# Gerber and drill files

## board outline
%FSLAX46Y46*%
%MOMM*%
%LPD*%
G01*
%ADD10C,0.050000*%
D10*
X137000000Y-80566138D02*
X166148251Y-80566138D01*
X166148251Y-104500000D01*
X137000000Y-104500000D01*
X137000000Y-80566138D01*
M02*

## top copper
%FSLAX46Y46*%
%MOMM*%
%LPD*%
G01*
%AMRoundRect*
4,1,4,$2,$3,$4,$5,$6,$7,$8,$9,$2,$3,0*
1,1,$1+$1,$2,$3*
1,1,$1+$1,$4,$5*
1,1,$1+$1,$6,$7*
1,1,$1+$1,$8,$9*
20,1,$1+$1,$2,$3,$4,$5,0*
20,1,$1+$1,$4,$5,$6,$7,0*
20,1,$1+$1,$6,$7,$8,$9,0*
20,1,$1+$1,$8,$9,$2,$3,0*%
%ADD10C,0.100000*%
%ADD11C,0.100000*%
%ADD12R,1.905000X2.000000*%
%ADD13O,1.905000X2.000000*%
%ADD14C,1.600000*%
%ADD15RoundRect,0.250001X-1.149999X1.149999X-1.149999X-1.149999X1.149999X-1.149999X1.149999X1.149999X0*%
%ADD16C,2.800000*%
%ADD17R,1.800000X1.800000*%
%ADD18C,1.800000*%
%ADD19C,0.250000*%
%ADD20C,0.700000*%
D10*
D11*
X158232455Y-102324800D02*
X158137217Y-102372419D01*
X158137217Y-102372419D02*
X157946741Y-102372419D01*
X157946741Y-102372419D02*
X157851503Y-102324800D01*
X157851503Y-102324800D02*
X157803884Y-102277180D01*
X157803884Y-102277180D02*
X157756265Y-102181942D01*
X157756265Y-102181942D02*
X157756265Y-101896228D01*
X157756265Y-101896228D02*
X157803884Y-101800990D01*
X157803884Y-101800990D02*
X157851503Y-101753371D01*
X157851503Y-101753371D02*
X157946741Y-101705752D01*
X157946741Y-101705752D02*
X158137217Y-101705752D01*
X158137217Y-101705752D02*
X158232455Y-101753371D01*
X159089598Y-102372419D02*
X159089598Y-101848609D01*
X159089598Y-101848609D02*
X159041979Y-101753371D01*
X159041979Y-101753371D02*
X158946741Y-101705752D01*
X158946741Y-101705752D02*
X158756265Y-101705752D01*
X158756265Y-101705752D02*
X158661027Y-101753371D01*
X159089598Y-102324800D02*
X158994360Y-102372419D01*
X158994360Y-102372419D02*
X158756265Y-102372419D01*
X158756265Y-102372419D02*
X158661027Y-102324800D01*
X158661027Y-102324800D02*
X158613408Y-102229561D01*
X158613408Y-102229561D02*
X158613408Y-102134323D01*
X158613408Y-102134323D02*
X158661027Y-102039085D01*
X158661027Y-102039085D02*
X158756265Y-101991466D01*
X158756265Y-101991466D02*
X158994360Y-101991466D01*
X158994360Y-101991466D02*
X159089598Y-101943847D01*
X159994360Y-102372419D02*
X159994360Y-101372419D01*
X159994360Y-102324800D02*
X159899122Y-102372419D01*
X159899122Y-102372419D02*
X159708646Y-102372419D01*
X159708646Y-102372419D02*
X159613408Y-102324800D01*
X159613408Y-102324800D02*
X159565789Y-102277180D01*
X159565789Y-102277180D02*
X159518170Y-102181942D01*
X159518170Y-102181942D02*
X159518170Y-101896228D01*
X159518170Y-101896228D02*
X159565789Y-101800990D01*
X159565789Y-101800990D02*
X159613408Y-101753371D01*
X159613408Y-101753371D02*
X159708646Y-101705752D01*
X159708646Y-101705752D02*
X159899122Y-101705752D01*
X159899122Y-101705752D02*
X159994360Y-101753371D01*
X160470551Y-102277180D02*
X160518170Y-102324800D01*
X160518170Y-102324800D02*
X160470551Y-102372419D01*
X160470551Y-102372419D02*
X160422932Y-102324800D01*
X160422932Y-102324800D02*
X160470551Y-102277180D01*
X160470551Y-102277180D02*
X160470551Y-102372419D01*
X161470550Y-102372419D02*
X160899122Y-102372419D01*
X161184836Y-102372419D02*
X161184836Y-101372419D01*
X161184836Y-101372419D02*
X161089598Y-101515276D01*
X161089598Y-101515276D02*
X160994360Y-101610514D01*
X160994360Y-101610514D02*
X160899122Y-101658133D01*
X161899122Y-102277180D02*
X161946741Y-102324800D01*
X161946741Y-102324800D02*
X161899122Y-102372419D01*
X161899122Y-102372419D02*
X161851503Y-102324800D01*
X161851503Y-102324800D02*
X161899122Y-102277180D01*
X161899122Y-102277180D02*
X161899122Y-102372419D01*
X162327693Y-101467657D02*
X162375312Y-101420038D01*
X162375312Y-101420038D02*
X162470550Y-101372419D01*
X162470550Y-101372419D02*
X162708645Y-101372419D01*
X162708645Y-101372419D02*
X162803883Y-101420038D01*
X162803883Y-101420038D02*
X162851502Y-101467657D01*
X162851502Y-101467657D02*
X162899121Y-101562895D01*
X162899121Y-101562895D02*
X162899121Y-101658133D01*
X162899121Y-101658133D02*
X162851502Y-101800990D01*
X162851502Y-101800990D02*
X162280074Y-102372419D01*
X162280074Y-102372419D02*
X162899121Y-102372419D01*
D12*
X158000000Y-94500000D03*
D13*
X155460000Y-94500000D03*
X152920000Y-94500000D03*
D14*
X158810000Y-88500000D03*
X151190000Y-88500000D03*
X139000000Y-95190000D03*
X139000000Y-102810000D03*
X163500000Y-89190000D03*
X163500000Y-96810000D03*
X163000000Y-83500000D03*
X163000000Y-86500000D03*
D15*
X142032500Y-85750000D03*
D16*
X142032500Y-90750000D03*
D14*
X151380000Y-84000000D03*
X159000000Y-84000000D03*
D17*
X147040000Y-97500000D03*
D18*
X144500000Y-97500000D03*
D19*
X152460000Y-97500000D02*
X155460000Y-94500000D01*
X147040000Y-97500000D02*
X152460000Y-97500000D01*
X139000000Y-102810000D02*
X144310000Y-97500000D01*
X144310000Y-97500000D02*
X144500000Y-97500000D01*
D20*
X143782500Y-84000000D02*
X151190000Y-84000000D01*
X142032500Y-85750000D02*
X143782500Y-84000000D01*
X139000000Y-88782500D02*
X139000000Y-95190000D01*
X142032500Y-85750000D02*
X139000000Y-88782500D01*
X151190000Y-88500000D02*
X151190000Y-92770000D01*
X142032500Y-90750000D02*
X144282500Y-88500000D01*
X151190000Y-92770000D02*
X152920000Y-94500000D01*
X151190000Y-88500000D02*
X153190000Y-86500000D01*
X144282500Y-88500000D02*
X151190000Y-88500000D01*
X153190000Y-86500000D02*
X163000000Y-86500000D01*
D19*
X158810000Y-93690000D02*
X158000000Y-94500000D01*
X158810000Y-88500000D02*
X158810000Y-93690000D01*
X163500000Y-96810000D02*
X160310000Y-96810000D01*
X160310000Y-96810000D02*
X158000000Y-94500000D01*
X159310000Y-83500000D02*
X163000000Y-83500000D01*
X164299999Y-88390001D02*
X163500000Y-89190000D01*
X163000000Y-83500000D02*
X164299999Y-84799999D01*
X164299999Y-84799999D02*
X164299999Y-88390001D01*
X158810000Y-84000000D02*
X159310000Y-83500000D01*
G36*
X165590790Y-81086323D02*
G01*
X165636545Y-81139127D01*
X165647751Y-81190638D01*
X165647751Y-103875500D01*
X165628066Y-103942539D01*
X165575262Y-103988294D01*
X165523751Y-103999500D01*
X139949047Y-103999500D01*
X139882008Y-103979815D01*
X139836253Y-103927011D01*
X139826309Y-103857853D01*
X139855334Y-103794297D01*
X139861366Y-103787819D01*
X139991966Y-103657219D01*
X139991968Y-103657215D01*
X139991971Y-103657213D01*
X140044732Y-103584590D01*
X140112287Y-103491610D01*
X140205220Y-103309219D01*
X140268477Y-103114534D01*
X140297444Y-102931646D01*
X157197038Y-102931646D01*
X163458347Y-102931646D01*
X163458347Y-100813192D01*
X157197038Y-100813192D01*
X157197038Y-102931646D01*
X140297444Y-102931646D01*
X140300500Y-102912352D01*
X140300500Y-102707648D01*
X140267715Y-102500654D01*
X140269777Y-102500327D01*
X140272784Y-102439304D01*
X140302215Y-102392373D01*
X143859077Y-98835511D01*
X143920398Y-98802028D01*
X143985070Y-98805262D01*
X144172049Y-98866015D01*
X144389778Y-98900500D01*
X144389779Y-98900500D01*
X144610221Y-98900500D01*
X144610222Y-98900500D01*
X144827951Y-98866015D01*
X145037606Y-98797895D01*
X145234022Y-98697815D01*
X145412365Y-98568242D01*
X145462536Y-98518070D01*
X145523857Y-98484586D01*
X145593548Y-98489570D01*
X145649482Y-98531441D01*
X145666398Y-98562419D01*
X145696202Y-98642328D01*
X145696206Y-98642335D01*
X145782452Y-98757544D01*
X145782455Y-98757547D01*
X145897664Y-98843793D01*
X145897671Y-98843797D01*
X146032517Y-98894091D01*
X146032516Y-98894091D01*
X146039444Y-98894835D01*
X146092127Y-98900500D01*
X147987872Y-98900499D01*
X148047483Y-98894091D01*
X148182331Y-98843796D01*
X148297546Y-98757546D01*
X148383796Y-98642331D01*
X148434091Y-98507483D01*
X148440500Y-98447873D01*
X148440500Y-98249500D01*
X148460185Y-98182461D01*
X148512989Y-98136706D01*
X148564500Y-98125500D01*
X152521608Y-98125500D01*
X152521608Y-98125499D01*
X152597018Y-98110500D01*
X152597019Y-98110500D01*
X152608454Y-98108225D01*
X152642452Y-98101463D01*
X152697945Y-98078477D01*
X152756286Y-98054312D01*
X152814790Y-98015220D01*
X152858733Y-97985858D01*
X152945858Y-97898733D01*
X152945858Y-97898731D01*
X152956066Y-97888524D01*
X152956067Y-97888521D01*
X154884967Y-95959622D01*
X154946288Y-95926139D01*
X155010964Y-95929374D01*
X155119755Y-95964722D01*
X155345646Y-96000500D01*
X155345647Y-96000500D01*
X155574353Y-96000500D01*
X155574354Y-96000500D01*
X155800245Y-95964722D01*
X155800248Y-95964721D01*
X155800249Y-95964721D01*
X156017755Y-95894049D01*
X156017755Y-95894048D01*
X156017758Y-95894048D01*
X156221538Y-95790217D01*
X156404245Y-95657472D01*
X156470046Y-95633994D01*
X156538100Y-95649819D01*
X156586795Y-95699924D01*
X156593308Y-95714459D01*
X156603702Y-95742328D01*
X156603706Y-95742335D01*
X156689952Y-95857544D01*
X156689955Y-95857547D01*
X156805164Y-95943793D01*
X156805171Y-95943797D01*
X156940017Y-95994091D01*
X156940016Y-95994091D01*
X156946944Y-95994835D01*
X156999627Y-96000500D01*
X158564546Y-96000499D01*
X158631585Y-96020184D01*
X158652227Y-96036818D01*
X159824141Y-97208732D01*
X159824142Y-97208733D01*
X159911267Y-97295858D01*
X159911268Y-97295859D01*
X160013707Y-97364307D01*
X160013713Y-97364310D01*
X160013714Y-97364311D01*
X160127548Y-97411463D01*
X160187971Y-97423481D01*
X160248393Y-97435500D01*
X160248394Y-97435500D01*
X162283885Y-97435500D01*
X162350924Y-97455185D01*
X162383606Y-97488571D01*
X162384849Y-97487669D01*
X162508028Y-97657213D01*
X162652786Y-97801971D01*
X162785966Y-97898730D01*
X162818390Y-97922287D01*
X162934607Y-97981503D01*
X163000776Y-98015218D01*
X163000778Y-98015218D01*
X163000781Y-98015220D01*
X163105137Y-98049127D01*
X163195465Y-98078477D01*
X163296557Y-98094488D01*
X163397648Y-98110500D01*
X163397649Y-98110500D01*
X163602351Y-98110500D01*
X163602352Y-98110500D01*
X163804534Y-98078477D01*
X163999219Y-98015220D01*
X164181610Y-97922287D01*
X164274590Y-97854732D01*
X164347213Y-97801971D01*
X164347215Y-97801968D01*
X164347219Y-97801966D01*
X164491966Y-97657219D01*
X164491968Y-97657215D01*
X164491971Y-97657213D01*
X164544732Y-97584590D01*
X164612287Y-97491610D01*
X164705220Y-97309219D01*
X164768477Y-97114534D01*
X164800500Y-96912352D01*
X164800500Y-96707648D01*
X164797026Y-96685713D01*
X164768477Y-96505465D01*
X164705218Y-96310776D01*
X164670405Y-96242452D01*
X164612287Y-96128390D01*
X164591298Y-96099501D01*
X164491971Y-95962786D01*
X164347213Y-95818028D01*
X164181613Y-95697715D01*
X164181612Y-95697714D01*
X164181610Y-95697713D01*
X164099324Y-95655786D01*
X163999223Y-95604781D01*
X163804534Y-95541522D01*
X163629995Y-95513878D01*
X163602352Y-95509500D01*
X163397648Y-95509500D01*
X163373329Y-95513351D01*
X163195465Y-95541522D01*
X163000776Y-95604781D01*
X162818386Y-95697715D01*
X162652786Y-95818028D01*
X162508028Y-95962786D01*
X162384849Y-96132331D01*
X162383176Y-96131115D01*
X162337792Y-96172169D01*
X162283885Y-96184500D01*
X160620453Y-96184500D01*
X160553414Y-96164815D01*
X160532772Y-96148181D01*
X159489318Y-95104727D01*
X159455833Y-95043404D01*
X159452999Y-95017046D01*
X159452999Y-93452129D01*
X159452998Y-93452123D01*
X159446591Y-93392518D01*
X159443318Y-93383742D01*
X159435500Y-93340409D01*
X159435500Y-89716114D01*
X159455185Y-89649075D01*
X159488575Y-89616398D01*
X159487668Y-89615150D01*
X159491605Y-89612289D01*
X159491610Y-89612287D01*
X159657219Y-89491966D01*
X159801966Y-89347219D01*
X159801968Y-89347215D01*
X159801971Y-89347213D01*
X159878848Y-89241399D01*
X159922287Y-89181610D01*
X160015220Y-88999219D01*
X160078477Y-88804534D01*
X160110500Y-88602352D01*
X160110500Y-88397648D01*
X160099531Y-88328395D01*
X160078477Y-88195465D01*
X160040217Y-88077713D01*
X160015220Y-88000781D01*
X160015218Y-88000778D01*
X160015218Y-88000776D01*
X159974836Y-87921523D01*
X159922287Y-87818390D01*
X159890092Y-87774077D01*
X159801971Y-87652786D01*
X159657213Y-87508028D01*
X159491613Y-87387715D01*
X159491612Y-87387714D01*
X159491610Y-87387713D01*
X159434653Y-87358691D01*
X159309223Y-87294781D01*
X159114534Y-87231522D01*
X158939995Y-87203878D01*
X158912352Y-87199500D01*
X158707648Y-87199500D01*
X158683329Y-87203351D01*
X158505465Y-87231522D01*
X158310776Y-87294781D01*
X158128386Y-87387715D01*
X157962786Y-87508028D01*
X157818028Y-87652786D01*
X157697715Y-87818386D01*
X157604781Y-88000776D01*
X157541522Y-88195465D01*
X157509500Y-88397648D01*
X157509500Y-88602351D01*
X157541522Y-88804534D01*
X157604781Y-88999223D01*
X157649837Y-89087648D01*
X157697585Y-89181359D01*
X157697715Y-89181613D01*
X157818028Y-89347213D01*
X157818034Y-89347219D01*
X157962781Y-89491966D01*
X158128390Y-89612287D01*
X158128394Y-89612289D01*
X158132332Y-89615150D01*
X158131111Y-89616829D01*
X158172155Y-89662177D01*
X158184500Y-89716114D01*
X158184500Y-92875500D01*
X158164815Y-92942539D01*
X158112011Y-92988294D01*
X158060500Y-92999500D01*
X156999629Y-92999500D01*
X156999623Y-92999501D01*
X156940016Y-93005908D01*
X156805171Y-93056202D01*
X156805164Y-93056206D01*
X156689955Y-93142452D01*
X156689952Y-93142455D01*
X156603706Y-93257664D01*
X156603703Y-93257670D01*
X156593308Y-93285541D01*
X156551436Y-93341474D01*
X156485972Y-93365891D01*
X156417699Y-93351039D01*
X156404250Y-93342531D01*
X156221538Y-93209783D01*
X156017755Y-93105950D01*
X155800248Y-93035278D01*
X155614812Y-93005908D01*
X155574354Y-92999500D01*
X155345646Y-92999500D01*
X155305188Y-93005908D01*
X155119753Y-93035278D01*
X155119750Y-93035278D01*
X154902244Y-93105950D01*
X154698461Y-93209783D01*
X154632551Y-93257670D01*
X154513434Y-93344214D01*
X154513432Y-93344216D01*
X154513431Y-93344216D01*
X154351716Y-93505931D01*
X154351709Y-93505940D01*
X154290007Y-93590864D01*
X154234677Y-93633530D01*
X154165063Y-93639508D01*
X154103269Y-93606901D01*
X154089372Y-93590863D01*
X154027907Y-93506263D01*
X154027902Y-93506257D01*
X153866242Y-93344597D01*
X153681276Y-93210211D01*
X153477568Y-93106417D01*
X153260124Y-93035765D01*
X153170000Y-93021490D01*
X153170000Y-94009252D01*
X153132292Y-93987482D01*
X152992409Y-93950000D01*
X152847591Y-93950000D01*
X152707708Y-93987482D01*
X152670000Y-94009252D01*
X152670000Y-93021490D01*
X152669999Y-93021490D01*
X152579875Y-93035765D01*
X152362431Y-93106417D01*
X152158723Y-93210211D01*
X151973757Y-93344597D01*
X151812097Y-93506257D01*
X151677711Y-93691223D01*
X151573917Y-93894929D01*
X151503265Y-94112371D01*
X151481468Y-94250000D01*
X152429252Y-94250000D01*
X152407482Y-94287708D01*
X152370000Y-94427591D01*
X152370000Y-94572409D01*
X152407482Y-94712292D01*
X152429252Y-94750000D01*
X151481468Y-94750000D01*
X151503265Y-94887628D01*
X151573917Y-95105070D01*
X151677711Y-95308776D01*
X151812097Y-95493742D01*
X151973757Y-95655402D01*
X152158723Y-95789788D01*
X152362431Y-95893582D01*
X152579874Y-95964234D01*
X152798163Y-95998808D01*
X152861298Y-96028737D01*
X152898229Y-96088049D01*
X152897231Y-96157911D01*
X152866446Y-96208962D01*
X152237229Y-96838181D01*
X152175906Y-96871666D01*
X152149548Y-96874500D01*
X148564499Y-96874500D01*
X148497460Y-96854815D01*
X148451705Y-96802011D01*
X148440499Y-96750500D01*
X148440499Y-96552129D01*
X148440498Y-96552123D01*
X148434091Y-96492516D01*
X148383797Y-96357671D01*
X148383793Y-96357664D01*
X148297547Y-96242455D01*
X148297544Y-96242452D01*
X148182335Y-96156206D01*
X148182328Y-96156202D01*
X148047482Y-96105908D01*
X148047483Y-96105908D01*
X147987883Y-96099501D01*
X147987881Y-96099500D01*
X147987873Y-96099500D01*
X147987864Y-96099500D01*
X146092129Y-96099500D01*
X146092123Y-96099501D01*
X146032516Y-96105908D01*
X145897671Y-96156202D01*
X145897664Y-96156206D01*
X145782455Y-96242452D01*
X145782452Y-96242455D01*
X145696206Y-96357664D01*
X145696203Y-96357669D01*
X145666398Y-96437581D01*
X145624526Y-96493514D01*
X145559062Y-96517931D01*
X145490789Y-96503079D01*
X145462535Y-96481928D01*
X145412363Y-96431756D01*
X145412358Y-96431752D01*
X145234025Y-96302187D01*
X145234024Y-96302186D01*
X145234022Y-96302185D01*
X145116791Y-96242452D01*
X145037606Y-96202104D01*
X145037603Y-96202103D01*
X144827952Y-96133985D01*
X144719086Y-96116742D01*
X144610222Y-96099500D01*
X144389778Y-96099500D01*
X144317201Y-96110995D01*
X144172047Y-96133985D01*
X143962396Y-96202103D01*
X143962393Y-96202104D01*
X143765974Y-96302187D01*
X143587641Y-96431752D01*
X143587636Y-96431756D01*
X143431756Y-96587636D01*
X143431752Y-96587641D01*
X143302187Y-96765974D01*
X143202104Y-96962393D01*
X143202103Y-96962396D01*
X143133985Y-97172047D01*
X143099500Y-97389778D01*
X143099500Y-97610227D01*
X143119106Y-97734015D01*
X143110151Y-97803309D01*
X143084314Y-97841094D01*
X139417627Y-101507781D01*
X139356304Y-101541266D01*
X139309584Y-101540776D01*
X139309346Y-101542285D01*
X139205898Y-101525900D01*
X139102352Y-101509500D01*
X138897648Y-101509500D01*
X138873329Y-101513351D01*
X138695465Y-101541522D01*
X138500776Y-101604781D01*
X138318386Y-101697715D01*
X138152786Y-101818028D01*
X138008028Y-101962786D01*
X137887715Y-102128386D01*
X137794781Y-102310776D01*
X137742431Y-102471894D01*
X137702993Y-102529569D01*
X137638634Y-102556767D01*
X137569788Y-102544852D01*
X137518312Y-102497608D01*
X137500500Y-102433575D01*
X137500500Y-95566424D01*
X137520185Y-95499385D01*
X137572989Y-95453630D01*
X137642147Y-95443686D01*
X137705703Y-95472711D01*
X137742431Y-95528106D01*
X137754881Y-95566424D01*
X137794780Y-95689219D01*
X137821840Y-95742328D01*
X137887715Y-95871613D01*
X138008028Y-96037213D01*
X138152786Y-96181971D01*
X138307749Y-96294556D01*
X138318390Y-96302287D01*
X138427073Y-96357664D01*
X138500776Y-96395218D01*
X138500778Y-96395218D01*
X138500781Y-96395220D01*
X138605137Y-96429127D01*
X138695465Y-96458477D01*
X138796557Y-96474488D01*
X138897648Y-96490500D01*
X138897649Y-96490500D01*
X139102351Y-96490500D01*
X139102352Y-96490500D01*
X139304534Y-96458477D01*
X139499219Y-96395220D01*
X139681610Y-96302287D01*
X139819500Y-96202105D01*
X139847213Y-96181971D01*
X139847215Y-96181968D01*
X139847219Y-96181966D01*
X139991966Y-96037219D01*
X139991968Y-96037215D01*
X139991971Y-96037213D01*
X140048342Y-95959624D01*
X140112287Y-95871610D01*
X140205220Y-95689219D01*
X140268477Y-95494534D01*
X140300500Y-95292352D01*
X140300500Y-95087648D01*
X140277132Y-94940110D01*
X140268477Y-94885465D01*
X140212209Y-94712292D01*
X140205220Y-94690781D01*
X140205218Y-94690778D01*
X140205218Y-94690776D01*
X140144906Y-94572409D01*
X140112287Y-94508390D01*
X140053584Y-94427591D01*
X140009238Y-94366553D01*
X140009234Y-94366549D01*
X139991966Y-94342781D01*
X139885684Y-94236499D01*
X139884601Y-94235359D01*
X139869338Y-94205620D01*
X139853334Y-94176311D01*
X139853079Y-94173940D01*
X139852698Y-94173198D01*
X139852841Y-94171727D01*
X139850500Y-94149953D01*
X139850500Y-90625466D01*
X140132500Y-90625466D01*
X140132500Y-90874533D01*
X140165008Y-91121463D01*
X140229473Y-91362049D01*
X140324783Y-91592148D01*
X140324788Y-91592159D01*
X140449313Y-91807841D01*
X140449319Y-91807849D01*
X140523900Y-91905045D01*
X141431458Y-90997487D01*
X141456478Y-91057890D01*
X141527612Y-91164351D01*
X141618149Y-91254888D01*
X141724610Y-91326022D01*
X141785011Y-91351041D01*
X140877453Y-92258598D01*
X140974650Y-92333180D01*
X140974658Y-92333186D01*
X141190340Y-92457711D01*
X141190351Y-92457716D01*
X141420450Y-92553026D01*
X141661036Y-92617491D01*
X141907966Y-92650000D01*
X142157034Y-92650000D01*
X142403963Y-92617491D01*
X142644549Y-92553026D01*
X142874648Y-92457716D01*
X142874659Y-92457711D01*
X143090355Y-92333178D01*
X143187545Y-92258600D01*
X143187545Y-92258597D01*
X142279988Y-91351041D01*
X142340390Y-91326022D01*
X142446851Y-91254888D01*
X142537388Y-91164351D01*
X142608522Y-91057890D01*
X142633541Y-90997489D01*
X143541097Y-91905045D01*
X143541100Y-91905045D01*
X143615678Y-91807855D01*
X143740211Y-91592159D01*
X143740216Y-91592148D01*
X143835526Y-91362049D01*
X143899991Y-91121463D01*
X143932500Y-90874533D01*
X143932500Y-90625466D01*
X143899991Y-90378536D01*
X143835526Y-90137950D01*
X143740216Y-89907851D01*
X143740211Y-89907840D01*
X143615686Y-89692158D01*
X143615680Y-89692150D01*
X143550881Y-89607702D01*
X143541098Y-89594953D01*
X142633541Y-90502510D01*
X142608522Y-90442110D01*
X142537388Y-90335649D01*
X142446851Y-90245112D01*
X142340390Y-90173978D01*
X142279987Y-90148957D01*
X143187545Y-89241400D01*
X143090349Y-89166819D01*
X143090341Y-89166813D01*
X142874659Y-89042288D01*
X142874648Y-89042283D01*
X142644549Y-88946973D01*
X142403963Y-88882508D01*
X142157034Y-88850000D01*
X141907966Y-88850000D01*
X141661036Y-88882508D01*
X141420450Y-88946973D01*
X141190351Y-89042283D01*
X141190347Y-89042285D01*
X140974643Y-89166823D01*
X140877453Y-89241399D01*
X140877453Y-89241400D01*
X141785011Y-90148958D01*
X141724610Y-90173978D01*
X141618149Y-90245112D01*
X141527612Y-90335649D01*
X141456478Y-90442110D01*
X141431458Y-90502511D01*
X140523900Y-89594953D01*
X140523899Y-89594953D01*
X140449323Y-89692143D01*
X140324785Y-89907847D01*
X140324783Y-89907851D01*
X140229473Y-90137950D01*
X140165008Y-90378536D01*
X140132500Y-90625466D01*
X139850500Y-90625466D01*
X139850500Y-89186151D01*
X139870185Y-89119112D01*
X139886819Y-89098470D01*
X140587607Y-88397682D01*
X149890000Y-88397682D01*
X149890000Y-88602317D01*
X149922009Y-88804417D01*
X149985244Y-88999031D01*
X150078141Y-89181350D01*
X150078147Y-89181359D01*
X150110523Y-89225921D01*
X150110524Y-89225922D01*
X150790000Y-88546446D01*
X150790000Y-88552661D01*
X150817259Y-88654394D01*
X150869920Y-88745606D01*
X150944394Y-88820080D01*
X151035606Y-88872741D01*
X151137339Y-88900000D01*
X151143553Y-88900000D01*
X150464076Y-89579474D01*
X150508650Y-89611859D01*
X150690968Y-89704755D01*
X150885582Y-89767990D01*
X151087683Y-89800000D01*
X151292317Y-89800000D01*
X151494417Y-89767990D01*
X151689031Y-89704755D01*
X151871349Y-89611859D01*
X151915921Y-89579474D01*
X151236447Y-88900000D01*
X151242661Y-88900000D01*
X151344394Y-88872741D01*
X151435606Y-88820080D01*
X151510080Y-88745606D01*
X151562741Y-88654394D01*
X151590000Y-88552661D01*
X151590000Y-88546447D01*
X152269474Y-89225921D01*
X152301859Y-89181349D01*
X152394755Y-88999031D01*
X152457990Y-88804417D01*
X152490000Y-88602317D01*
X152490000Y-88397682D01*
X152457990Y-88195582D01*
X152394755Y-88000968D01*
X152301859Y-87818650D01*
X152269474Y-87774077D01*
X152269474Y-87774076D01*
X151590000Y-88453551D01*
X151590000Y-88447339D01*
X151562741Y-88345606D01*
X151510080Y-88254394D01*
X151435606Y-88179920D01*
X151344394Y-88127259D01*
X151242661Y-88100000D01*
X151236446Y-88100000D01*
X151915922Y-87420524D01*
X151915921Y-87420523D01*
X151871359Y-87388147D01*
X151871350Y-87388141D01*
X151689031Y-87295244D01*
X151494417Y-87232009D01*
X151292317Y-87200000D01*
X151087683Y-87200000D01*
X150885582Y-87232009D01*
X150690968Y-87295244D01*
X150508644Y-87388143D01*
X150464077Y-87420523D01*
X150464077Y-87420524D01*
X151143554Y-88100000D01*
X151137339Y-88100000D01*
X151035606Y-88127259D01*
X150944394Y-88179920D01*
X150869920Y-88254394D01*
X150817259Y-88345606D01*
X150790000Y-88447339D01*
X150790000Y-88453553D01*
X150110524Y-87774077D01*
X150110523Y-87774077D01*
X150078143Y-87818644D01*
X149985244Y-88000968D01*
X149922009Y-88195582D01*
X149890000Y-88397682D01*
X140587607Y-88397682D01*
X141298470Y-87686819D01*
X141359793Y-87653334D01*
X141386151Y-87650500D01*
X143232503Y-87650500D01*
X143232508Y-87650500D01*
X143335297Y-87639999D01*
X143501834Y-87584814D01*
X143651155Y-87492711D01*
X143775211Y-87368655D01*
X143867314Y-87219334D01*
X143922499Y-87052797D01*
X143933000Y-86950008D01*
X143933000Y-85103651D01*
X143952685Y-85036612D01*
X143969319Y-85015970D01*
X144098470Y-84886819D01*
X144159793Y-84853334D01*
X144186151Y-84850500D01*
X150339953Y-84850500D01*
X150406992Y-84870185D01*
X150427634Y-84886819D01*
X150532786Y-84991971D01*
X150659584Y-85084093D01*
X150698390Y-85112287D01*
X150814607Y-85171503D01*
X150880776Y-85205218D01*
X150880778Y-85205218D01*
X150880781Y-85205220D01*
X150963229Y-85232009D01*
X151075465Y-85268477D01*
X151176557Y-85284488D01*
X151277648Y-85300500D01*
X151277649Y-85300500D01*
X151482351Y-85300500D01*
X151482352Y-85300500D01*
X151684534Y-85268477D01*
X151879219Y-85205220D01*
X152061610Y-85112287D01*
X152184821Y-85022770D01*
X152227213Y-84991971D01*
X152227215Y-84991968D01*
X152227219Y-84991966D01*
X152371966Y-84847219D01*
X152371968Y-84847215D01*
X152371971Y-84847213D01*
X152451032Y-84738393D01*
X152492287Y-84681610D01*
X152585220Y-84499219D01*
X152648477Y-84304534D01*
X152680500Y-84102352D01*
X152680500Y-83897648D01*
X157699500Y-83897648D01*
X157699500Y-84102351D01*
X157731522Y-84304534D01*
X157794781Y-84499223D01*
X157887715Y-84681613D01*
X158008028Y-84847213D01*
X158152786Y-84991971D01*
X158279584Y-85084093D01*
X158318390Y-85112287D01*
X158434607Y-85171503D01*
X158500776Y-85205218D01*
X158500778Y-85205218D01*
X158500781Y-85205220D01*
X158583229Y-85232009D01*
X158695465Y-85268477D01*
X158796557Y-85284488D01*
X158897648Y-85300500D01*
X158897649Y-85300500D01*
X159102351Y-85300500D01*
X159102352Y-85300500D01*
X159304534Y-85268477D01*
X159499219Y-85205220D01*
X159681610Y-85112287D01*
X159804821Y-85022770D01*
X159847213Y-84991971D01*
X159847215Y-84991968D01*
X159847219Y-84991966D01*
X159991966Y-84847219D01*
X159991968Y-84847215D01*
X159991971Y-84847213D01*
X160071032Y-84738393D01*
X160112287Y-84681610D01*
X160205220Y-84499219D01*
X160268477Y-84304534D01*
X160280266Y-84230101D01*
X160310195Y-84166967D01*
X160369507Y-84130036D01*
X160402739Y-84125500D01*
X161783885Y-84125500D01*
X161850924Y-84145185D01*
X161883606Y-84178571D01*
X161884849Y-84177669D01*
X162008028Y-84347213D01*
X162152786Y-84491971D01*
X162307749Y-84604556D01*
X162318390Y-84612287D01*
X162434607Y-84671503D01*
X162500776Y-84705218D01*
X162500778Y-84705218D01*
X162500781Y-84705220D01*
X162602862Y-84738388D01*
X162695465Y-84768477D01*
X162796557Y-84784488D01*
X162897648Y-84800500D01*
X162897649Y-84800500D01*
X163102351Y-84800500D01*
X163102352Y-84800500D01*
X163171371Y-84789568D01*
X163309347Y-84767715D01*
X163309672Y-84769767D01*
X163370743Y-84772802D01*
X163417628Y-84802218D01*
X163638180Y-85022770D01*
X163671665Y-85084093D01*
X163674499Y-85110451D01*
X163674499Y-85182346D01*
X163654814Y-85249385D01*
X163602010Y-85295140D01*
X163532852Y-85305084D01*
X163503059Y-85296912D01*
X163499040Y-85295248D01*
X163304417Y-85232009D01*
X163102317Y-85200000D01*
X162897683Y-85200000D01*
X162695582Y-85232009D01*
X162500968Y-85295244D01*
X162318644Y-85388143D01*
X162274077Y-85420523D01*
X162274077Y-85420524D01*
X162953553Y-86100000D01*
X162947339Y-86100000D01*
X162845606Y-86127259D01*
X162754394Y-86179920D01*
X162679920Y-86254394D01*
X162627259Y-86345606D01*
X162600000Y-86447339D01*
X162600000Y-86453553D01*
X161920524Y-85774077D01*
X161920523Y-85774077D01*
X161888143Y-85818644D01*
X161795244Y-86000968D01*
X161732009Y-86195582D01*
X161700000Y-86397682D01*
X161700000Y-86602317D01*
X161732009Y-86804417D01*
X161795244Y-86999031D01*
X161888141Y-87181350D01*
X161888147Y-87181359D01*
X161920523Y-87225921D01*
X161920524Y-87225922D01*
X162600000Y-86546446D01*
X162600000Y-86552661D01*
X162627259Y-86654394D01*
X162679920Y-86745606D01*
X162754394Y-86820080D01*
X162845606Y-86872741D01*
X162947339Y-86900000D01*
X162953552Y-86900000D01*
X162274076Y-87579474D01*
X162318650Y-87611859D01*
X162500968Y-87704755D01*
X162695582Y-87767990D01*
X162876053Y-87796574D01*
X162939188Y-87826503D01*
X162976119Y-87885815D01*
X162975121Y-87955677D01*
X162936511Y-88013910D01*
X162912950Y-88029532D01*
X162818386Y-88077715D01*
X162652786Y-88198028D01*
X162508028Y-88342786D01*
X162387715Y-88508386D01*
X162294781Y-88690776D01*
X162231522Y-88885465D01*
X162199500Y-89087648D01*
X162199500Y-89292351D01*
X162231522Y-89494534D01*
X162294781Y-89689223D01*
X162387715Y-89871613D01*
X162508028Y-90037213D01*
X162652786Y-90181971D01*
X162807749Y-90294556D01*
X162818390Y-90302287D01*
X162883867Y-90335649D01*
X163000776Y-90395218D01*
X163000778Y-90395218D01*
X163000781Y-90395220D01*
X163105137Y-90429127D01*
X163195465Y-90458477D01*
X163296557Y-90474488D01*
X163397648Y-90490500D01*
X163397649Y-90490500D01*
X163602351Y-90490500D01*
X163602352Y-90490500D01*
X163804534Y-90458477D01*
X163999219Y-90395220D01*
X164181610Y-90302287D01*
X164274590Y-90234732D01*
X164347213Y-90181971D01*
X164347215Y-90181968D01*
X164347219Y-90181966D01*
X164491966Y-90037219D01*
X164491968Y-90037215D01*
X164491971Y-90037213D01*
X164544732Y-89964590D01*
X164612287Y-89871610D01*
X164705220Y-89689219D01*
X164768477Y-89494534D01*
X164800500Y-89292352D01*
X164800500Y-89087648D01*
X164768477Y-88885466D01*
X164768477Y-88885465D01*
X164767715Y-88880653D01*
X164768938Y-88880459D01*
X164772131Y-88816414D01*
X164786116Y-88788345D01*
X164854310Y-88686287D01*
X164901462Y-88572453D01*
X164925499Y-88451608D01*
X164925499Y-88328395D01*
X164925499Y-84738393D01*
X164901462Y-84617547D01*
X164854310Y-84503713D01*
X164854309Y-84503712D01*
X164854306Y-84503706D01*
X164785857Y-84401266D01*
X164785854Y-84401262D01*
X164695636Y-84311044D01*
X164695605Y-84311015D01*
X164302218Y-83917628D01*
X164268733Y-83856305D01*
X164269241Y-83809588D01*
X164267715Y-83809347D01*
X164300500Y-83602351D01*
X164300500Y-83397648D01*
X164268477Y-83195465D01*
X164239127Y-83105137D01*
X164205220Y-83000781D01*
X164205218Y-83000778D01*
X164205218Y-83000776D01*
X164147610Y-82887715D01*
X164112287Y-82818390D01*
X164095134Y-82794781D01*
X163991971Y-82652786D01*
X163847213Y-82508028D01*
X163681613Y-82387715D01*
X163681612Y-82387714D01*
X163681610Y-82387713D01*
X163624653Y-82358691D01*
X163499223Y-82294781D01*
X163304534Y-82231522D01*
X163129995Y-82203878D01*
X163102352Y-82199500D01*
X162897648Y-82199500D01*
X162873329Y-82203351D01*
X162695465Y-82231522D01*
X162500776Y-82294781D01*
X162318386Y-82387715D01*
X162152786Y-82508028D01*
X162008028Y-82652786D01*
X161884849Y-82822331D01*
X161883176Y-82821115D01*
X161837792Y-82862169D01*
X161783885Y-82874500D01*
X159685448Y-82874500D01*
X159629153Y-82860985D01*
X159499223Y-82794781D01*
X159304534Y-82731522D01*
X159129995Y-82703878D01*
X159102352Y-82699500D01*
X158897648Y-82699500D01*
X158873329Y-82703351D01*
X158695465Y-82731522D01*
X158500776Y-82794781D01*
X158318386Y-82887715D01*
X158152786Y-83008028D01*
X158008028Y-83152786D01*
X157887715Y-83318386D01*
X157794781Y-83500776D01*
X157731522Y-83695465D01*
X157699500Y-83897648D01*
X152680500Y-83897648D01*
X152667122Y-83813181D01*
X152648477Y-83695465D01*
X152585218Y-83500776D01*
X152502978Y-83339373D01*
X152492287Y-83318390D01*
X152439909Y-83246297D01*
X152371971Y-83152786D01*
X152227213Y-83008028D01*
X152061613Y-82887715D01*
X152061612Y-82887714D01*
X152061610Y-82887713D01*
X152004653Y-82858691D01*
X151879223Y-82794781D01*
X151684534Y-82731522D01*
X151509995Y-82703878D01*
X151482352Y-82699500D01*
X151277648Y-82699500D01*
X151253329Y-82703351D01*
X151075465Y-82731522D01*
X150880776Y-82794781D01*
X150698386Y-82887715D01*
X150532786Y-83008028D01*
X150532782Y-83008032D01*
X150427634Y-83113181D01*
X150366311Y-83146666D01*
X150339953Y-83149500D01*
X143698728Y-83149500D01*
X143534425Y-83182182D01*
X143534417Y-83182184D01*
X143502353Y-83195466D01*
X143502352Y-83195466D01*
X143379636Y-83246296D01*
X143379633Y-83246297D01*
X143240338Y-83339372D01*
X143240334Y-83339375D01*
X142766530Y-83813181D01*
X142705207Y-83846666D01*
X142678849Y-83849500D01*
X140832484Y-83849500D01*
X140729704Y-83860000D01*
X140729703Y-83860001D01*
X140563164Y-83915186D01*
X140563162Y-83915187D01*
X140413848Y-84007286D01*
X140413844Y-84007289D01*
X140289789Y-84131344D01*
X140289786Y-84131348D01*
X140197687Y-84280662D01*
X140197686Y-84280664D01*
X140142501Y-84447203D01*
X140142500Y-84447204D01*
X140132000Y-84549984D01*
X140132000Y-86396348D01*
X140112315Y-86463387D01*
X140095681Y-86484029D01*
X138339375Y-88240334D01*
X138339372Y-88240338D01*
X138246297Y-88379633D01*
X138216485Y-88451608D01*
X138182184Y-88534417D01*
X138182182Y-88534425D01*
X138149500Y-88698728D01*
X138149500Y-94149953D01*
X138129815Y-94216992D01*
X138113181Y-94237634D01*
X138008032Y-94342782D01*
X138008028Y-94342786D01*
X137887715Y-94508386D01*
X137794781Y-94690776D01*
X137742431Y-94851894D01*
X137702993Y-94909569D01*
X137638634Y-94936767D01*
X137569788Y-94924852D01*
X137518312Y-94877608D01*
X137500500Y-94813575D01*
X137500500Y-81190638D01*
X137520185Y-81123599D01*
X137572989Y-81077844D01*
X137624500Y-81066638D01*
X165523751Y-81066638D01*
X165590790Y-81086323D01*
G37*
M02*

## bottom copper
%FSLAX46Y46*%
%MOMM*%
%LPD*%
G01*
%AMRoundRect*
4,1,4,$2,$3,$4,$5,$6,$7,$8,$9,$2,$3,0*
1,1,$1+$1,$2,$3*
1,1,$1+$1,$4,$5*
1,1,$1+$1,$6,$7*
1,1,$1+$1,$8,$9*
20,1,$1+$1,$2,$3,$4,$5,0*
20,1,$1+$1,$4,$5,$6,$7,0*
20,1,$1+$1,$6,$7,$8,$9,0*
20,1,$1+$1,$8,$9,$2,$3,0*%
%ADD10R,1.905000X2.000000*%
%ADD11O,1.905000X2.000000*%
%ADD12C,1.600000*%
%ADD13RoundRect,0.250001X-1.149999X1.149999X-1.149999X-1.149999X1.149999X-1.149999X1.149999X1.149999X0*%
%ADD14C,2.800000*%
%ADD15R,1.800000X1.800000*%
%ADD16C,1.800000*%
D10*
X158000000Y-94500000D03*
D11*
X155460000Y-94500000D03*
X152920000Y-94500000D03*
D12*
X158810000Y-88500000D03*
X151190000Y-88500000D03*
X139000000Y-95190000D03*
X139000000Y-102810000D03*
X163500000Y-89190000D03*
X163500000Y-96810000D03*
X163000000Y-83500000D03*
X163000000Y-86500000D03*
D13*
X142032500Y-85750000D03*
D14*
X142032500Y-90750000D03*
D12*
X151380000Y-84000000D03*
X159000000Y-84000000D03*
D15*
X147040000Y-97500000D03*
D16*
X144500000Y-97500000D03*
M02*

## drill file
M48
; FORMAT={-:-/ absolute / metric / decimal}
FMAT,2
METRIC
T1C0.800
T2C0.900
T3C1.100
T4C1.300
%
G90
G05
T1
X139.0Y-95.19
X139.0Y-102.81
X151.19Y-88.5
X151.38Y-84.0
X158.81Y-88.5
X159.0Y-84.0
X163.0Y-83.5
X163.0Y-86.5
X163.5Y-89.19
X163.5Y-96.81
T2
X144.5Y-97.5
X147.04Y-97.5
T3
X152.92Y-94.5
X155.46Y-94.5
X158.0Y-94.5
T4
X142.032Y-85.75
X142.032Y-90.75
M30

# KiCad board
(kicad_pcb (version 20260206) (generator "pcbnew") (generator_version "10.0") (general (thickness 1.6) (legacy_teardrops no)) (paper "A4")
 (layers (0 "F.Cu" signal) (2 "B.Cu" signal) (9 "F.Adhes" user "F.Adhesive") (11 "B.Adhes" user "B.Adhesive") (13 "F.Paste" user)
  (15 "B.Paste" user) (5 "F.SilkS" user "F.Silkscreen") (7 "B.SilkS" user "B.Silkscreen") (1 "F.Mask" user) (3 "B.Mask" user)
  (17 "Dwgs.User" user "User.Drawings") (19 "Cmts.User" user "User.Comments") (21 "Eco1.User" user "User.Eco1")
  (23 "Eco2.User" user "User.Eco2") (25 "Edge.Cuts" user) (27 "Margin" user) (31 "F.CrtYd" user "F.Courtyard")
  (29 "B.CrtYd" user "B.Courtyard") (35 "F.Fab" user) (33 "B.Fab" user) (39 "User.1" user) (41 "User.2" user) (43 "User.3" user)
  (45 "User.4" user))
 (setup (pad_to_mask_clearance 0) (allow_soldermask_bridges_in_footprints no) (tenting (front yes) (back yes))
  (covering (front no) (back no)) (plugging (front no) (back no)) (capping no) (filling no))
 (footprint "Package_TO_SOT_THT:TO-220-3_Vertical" (layer "F.Cu") (at 158 94.5 180)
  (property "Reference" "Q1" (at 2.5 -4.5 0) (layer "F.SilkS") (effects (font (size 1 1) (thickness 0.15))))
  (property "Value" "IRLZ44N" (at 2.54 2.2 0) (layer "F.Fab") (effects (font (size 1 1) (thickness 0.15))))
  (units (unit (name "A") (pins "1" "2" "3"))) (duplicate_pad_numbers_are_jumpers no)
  (pad "1" thru_hole rect (at 0 0 180) (size 1.905 2) (drill 1.1) (layers "*.Cu" "*.Mask") (remove_unused_layers no) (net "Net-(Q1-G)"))
  (pad "2" thru_hole oval (at 2.54 0 180) (size 1.905 2) (drill 1.1) (layers "*.Cu" "*.Mask") (remove_unused_layers no) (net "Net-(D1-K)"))
  (pad "3" thru_hole oval (at 5.08 0 180) (size 1.905 2) (drill 1.1) (layers "*.Cu" "*.Mask") (remove_unused_layers no) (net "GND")))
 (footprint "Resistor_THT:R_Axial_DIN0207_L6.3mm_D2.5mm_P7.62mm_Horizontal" (layer "F.Cu") (at 158.81 88.5 180)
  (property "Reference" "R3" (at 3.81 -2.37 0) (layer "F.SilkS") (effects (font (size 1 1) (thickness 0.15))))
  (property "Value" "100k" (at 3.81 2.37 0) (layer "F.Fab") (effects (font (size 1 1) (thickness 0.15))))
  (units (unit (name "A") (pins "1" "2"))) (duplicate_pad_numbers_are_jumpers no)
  (pad "1" thru_hole circle (at 0 0 180) (size 1.6 1.6) (drill 0.8) (layers "*.Cu" "*.Mask") (remove_unused_layers no) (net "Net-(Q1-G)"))
  (pad "2" thru_hole circle (at 7.62 0 180) (size 1.6 1.6) (drill 0.8) (layers "*.Cu" "*.Mask") (remove_unused_layers no) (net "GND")))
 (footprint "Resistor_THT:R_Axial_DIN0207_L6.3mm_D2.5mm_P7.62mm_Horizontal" (layer "F.Cu") (at 139 95.19 -90)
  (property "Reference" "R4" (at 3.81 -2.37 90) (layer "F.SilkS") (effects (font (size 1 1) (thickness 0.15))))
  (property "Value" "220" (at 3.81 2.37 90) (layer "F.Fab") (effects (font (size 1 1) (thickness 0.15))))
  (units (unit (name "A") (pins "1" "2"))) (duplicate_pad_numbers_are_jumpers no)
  (pad "1" thru_hole circle (at 0 0 270) (size 1.6 1.6) (drill 0.8) (layers "*.Cu" "*.Mask") (remove_unused_layers no) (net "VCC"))
  (pad "2" thru_hole circle (at 7.62 0 270) (size 1.6 1.6) (drill 0.8) (layers "*.Cu" "*.Mask") (remove_unused_layers no) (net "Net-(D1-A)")))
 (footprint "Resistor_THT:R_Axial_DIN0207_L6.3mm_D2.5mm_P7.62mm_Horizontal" (layer "F.Cu") (at 163.5 89.19 -90)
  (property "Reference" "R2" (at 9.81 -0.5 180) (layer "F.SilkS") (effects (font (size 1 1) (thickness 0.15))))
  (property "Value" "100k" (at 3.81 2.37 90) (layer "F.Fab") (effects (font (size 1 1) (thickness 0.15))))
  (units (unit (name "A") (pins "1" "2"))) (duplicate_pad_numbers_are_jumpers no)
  (pad "1" thru_hole circle (at 0 0 270) (size 1.6 1.6) (drill 0.8) (layers "*.Cu" "*.Mask") (remove_unused_layers no) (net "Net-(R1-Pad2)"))
  (pad "2" thru_hole circle (at 7.62 0 270) (size 1.6 1.6) (drill 0.8) (layers "*.Cu" "*.Mask") (remove_unused_layers no) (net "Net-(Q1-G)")))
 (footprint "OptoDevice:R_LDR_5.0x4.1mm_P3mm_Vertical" (layer "F.Cu") (at 163 83.5 -90)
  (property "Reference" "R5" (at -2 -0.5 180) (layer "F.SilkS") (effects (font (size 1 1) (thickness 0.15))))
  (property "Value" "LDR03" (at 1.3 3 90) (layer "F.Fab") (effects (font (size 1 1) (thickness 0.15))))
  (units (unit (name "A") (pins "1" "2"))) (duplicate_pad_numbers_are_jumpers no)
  (pad "1" thru_hole circle (at 0 0 270) (size 1.6 1.6) (drill 0.8) (layers "*.Cu" "*.Mask") (remove_unused_layers no) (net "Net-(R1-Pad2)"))
  (pad "2" thru_hole circle (at 3 0 270) (size 1.6 1.6) (drill 0.8) (layers "*.Cu" "*.Mask") (remove_unused_layers no) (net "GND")))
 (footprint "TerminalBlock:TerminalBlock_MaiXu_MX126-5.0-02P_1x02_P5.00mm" (layer "F.Cu") (at 142.0325 85.75 -90)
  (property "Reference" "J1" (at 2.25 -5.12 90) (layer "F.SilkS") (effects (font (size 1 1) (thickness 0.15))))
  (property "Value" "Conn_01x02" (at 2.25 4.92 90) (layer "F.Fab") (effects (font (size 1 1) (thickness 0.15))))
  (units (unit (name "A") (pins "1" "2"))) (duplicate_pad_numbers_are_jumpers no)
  (pad "1" thru_hole roundrect (at 0 0 270) (size 2.8 2.8) (drill 1.3) (layers "*.Cu" "*.Mask") (remove_unused_layers no)
   (roundrect_rratio 0.089286) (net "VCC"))
  (pad "2" thru_hole circle (at 5 0 270) (size 2.8 2.8) (drill 1.3) (layers "*.Cu" "*.Mask") (remove_unused_layers no) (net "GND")))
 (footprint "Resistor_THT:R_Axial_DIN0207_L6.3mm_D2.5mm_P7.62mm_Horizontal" (layer "F.Cu") (at 151.38 84)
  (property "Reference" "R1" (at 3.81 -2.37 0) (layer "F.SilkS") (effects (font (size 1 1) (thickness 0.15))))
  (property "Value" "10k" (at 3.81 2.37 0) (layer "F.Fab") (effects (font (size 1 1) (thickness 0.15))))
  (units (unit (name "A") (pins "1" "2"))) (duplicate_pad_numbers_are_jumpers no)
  (pad "1" thru_hole circle (at 0 0) (size 1.6 1.6) (drill 0.8) (layers "*.Cu" "*.Mask") (remove_unused_layers no) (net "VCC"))
  (pad "2" thru_hole circle (at 7.62 0) (size 1.6 1.6) (drill 0.8) (layers "*.Cu" "*.Mask") (remove_unused_layers no) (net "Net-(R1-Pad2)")))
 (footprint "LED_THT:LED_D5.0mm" (layer "F.Cu") (at 147.04 97.5 180)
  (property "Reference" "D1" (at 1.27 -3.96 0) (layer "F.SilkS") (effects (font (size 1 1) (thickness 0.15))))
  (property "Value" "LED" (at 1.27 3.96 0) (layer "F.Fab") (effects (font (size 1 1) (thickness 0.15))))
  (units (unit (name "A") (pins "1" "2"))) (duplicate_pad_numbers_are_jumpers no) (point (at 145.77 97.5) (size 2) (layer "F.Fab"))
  (pad "1" thru_hole rect (at 0 0 180) (size 1.8 1.8) (drill 0.9) (layers "*.Cu" "*.Mask") (remove_unused_layers no) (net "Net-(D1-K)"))
  (pad "2" thru_hole circle (at 2.54 0 180) (size 1.8 1.8) (drill 0.9) (layers "*.Cu" "*.Mask") (remove_unused_layers no) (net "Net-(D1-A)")))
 (gr_rect (start 137 80.566138) (end 166.148251 104.5) (stroke (width 0.05) (type default)) (fill no) (layer "Edge.Cuts"))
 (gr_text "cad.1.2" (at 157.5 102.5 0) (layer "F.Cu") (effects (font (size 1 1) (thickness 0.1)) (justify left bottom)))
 (segment (start 152.46 97.5) (end 155.46 94.5) (width 0.25) (layer "F.Cu") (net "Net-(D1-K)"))
 (segment (start 147.04 97.5) (end 152.46 97.5) (width 0.25) (layer "F.Cu") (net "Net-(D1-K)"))
 (segment (start 139 102.81) (end 144.31 97.5) (width 0.25) (layer "F.Cu") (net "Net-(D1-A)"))
 (segment (start 144.31 97.5) (end 144.5 97.5) (width 0.25) (layer "F.Cu") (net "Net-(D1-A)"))
 (segment (start 143.7825 84) (end 151.19 84) (width 0.7) (layer "F.Cu") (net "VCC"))
 (segment (start 142.0325 85.75) (end 143.7825 84) (width 0.7) (layer "F.Cu") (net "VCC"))
 (segment (start 139 88.7825) (end 139 95.19) (width 0.7) (layer "F.Cu") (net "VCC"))
 (segment (start 142.0325 85.75) (end 139 88.7825) (width 0.7) (layer "F.Cu") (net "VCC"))
 (segment (start 151.19 88.5) (end 151.19 92.77) (width 0.7) (layer "F.Cu") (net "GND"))
 (segment (start 142.0325 90.75) (end 144.2825 88.5) (width 0.7) (layer "F.Cu") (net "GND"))
 (segment (start 151.19 92.77) (end 152.92 94.5) (width 0.7) (layer "F.Cu") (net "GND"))
 (segment (start 151.19 88.5) (end 153.19 86.5) (width 0.7) (layer "F.Cu") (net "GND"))
 (segment (start 144.2825 88.5) (end 151.19 88.5) (width 0.7) (layer "F.Cu") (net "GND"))
 (segment (start 153.19 86.5) (end 163 86.5) (width 0.7) (layer "F.Cu") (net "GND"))
 (segment (start 158.81 93.69) (end 158 94.5) (width 0.25) (layer "F.Cu") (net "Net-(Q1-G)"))
 (segment (start 158.81 88.5) (end 158.81 93.69) (width 0.25) (layer "F.Cu") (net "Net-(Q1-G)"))
 (segment (start 163.5 96.81) (end 160.31 96.81) (width 0.25) (layer "F.Cu") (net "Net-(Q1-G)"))
 (segment (start 160.31 96.81) (end 158 94.5) (width 0.25) (layer "F.Cu") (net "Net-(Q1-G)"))
 (segment (start 159.31 83.5) (end 163 83.5) (width 0.25) (layer "F.Cu") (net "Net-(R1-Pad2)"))
 (segment (start 164.299999 88.390001) (end 163.5 89.19) (width 0.25) (layer "F.Cu") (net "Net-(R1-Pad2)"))
 (segment (start 163 83.5) (end 164.299999 84.799999) (width 0.25) (layer "F.Cu") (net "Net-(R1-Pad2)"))
 (segment (start 164.299999 84.799999) (end 164.299999 88.390001) (width 0.25) (layer "F.Cu") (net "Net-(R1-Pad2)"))
 (segment (start 158.81 84) (end 159.31 83.5) (width 0.25) (layer "F.Cu") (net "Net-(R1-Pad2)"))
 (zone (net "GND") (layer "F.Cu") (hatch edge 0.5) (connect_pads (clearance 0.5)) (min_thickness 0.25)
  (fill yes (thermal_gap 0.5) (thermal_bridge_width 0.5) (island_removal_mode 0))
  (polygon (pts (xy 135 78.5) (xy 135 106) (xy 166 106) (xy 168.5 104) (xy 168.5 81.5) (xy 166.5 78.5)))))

